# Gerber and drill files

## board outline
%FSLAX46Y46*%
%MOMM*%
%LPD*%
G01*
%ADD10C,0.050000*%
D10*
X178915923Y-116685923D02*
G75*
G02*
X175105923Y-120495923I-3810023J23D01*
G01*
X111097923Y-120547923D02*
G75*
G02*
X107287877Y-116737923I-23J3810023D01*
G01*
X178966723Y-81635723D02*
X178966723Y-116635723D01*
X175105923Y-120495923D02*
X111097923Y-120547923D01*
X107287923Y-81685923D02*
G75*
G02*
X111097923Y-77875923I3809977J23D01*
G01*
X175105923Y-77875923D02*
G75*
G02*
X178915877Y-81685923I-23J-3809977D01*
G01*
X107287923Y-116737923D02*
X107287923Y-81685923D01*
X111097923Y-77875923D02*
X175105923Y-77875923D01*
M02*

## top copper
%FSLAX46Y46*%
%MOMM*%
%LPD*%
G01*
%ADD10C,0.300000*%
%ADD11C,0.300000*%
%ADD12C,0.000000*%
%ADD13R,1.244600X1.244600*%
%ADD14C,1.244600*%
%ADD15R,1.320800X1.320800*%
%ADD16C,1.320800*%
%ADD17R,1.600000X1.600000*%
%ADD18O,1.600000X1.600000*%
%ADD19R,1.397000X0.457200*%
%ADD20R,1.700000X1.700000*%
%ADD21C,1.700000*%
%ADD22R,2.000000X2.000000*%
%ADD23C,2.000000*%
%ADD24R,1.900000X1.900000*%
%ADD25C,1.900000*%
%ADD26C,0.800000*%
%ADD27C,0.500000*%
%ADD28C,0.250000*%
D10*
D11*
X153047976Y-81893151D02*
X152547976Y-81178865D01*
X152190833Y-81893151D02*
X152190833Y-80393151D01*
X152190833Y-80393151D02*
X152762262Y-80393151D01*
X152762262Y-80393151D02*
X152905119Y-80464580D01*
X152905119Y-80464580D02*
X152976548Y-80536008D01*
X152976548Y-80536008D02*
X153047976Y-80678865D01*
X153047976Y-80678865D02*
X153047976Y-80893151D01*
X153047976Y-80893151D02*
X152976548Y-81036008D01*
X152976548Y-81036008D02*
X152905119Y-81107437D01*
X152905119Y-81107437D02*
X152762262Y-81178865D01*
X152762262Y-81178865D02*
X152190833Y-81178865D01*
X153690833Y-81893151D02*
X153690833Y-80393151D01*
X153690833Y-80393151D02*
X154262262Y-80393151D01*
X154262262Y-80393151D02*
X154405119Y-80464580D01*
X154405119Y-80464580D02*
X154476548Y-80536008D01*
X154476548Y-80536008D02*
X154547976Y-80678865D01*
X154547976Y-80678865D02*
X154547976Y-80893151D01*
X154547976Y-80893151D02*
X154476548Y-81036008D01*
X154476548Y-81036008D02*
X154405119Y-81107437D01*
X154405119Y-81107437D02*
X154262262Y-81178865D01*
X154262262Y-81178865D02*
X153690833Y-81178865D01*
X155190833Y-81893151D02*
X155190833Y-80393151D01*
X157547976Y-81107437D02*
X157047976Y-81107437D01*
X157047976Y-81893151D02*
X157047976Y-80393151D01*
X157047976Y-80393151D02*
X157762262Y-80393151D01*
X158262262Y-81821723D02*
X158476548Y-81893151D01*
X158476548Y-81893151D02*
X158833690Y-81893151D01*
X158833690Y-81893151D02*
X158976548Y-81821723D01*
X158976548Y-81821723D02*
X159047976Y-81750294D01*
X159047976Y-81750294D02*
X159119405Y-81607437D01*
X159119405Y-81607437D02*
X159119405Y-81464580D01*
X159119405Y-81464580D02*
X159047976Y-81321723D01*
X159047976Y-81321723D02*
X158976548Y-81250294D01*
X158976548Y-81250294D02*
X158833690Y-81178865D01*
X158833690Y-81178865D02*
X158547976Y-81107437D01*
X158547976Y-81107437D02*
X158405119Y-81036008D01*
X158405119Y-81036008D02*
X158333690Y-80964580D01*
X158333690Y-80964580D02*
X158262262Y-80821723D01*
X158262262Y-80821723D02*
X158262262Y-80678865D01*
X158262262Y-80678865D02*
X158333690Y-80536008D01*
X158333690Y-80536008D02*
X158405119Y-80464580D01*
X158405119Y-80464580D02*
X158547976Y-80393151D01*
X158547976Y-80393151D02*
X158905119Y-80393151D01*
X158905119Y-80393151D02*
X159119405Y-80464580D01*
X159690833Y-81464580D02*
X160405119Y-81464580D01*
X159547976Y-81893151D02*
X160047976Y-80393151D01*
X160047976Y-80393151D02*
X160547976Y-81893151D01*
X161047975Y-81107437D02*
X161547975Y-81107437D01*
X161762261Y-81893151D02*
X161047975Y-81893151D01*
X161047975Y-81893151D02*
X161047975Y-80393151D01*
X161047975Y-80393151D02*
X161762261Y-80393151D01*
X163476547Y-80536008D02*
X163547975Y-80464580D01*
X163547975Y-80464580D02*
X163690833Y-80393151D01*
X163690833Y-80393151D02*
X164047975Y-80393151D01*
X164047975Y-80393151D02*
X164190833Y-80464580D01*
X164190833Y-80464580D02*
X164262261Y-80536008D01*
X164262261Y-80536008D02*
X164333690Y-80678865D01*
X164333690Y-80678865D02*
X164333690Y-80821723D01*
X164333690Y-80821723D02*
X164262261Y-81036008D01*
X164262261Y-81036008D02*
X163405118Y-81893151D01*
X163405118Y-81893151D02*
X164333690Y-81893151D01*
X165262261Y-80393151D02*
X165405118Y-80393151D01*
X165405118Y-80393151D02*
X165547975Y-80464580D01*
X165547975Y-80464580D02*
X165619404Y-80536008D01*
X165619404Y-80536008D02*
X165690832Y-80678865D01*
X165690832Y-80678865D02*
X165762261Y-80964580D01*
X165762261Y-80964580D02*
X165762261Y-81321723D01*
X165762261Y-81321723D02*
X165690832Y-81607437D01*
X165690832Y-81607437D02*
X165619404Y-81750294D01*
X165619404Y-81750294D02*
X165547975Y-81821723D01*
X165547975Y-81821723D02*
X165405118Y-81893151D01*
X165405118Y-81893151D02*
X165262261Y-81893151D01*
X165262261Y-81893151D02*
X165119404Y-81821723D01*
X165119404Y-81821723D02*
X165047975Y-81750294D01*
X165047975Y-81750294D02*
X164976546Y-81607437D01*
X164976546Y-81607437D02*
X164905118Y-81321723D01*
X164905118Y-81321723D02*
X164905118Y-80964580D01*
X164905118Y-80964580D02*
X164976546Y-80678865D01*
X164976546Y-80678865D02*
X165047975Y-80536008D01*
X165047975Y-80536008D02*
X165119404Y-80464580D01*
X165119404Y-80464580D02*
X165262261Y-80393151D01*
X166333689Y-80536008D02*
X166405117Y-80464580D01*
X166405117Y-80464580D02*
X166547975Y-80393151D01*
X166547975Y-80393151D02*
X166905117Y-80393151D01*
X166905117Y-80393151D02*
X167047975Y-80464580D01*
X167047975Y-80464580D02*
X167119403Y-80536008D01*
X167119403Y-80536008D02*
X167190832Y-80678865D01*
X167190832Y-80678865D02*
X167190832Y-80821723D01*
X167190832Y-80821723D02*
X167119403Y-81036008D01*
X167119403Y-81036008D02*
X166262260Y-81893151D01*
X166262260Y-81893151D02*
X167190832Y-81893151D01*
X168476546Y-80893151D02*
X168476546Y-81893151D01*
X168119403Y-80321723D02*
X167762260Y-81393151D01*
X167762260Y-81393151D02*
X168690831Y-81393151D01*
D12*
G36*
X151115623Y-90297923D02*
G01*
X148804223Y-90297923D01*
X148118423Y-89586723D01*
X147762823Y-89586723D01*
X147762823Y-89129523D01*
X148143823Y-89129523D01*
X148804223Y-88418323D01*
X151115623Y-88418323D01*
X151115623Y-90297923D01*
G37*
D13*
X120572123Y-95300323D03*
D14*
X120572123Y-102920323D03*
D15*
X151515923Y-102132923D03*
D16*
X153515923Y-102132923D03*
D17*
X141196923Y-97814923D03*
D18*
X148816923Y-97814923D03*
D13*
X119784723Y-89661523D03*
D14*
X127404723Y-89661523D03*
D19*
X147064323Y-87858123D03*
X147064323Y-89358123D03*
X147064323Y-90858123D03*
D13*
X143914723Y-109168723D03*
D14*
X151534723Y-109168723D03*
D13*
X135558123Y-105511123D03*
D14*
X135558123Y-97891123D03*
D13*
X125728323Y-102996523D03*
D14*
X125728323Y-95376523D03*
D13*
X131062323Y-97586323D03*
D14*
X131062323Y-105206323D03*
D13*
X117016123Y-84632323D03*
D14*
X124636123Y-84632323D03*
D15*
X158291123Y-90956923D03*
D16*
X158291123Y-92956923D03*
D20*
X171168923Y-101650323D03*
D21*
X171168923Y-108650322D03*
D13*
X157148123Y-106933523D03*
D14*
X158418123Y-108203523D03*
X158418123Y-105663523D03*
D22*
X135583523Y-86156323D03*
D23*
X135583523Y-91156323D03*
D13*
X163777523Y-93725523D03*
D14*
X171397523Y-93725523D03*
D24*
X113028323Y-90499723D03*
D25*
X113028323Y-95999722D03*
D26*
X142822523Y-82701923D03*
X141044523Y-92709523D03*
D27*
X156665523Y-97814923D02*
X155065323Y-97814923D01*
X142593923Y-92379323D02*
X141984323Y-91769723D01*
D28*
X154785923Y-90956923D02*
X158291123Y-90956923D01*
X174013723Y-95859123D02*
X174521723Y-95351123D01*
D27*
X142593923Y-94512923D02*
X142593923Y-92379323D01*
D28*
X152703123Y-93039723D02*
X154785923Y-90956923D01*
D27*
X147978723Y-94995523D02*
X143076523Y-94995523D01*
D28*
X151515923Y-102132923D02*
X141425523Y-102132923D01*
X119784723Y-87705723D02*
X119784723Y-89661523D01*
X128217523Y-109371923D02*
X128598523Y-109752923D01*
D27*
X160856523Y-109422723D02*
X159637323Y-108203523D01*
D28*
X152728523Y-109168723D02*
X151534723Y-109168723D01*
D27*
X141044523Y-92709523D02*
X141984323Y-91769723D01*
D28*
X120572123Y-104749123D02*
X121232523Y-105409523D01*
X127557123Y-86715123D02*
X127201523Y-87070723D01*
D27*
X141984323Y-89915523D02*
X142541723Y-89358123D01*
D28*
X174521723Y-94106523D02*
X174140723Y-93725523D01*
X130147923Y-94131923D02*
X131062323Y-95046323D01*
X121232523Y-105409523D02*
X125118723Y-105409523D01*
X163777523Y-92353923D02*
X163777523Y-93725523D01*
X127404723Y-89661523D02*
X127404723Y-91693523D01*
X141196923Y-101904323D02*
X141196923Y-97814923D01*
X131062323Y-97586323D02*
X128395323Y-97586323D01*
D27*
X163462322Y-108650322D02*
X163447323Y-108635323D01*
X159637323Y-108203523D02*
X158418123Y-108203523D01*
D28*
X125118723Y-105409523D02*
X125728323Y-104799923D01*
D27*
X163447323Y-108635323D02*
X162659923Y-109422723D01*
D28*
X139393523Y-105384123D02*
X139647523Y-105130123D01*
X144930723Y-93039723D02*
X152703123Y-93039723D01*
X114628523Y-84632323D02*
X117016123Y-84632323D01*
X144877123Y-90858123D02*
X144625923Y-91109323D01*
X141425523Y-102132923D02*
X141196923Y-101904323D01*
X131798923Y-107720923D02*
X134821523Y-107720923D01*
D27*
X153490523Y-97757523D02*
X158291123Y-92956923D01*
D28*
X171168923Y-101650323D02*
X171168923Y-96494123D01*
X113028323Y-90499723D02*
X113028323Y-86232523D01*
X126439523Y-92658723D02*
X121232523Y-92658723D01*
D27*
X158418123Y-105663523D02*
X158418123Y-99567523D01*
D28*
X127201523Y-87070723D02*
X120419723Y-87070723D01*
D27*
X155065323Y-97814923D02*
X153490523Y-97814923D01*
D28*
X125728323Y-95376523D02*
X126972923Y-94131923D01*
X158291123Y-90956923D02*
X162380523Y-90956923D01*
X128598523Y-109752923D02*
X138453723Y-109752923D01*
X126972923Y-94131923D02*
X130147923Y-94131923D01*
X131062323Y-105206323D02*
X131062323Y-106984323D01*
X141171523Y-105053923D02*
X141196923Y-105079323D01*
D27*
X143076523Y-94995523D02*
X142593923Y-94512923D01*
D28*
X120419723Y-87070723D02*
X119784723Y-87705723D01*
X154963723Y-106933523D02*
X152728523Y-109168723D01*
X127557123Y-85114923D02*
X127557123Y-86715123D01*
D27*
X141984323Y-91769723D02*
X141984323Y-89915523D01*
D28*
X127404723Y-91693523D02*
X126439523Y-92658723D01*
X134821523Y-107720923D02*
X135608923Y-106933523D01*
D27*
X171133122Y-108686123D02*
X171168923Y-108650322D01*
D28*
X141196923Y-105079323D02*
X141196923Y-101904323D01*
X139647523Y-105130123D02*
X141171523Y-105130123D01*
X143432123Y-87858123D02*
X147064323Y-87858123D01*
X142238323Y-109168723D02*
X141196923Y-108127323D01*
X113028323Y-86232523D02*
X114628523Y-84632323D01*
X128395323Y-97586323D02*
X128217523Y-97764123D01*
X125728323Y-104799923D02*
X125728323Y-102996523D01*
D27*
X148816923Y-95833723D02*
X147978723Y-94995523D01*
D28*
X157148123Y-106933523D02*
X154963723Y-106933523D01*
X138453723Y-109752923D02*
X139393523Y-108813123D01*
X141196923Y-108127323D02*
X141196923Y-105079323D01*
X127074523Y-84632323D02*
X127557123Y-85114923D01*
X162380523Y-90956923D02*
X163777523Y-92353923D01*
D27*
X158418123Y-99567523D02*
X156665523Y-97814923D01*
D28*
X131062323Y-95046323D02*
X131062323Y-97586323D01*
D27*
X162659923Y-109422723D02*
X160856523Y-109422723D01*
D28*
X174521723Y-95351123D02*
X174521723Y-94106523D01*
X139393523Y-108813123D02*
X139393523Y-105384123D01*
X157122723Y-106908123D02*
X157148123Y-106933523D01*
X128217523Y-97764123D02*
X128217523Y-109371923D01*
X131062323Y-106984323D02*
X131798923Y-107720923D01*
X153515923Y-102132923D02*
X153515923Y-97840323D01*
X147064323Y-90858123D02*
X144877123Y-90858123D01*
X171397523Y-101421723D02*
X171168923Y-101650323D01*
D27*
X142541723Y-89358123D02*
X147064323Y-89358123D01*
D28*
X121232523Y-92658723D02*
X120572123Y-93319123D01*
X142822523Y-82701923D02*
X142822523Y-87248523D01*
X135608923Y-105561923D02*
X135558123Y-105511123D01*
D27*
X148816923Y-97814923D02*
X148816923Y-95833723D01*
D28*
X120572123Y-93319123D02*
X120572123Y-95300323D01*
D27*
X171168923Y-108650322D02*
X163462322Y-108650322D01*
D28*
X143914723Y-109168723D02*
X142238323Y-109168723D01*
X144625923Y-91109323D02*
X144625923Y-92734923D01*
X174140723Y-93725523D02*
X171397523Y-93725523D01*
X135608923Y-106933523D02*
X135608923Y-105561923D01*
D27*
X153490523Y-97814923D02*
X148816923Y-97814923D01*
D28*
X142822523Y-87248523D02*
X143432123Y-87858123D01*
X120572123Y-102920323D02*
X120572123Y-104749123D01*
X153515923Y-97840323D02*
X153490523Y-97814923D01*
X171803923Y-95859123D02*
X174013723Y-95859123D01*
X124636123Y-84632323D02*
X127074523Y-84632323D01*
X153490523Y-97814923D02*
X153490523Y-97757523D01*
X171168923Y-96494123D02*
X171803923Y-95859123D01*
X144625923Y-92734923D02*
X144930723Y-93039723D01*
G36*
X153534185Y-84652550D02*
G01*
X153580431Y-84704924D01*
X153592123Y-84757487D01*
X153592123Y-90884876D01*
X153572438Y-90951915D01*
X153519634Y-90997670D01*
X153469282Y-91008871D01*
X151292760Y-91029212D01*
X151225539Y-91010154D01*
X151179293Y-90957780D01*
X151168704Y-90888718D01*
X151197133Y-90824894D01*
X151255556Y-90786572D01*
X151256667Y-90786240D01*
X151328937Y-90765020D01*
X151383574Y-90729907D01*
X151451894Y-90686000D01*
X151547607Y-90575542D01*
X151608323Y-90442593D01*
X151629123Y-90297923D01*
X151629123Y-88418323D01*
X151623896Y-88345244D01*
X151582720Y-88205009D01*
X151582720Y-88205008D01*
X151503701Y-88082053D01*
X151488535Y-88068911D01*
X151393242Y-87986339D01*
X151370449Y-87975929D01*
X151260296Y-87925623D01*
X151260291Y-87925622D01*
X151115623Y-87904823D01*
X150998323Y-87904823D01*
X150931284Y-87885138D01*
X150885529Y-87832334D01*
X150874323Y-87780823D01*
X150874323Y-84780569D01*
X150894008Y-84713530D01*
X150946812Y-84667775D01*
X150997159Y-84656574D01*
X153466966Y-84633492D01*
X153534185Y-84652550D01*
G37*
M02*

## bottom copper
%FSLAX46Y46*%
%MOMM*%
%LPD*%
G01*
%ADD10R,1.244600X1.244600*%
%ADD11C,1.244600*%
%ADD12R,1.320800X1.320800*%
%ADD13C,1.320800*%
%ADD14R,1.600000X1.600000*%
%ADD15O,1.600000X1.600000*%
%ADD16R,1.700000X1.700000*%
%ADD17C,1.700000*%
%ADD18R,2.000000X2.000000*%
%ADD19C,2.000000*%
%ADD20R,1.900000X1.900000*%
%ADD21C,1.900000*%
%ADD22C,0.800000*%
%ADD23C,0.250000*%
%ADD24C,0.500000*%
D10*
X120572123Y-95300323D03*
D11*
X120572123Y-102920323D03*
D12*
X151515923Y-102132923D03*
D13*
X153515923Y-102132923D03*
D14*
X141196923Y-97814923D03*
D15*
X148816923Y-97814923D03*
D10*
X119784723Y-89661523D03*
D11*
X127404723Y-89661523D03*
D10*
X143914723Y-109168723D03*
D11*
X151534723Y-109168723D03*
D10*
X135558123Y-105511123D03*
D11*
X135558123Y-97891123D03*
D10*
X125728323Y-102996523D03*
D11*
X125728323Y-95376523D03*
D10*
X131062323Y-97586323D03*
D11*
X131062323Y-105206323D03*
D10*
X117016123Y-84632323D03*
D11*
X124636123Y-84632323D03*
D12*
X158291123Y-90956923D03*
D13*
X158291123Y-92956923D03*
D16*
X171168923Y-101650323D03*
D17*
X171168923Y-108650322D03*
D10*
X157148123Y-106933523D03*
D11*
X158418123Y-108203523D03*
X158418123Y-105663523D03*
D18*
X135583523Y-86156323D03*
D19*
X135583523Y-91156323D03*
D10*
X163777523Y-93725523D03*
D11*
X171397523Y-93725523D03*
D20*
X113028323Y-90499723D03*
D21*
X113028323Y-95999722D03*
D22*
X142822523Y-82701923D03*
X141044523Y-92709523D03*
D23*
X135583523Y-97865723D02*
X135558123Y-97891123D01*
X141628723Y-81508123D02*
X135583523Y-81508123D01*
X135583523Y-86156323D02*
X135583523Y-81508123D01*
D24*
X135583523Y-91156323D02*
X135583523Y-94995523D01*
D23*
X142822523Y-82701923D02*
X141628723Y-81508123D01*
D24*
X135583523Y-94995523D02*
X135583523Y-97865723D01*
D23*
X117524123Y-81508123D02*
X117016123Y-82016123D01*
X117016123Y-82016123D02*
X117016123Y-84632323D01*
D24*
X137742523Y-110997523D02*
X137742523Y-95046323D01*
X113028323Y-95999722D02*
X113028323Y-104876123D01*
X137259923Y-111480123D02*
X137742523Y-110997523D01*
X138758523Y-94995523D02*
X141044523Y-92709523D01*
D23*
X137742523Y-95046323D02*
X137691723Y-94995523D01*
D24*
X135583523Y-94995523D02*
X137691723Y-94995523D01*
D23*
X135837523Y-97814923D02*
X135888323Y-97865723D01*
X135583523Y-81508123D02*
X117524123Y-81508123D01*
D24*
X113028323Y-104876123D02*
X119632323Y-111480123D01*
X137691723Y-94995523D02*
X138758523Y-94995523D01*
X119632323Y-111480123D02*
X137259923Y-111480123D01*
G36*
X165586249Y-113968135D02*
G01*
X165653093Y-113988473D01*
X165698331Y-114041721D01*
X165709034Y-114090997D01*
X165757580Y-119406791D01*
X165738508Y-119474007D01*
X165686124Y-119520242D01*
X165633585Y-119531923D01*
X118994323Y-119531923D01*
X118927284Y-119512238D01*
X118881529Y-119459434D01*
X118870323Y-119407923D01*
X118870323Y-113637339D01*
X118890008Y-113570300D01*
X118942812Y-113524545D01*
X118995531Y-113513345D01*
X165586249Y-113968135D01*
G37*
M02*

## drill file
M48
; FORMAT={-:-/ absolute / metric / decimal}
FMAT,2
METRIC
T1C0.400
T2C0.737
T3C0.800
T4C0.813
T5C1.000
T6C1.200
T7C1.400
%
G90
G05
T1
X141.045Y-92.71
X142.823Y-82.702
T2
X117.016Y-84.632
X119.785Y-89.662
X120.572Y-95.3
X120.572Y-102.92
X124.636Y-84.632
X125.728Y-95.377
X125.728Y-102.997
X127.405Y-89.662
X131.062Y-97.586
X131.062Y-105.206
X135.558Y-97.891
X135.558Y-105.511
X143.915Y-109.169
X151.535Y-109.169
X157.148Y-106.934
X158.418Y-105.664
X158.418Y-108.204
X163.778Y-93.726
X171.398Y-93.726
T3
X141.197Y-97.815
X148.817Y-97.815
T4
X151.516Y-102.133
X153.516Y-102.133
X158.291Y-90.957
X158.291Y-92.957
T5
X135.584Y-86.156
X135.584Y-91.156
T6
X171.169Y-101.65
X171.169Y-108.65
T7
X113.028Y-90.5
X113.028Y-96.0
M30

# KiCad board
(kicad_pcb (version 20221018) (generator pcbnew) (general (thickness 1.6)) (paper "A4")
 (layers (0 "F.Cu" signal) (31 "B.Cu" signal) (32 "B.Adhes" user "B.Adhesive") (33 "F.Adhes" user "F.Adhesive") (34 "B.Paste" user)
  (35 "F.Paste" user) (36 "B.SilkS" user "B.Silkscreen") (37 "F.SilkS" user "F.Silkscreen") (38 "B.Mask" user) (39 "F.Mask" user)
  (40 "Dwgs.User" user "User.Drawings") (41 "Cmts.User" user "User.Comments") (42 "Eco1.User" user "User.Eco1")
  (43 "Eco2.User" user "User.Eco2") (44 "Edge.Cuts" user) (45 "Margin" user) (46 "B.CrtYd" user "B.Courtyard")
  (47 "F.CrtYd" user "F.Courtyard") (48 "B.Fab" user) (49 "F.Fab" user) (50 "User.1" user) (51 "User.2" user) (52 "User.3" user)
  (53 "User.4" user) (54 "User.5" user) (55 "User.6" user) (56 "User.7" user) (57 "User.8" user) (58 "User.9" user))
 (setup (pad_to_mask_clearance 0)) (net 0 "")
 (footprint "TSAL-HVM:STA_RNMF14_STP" (layer "F.Cu") (at 120.572123 95.300323 -90)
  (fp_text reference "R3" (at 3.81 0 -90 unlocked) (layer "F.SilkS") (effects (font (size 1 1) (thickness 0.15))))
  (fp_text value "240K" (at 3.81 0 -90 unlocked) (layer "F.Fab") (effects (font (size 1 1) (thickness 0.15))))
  (pad "1" thru_hole rect (at 0 0 270) (size 1.2446 1.2446) (drill 0.7366) (layers "*.Cu" "*.Mask"))
  (pad "2" thru_hole circle (at 7.62 0 270) (size 1.2446 1.2446) (drill 0.7366) (layers "*.Cu" "*.Mask")))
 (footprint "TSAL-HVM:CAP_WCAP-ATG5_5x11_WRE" (layer "F.Cu") (at 151.515923 102.132923)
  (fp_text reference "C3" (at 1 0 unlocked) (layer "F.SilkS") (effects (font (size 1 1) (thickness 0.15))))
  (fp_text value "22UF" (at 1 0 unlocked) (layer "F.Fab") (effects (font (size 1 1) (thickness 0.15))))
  (pad "1" thru_hole rect (at 0 0) (size 1.3208 1.3208) (drill 0.8128) (layers "*.Cu" "*.Mask"))
  (pad "2" thru_hole circle (at 2 0) (size 1.3208 1.3208) (drill 0.8128) (layers "*.Cu" "*.Mask")))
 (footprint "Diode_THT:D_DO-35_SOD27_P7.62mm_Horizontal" (layer "F.Cu") (at 141.196923 97.814923)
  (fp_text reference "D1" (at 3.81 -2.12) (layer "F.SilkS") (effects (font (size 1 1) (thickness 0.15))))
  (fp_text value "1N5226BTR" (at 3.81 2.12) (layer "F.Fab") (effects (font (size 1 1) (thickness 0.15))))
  (pad "1" thru_hole rect (at 0 0) (size 1.6 1.6) (drill 0.8) (layers "*.Cu" "*.Mask"))
  (pad "2" thru_hole oval (at 7.62 0) (size 1.6 1.6) (drill 0.8) (layers "*.Cu" "*.Mask")))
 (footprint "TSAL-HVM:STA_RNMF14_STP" (layer "F.Cu") (at 119.784723 89.661523)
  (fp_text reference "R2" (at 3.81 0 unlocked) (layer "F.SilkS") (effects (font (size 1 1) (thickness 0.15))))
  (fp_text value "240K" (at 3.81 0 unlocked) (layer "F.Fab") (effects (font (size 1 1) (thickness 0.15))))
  (pad "1" thru_hole rect (at 0 0) (size 1.2446 1.2446) (drill 0.7366) (layers "*.Cu" "*.Mask"))
  (pad "2" thru_hole circle (at 7.62 0) (size 1.2446 1.2446) (drill 0.7366) (layers "*.Cu" "*.Mask")))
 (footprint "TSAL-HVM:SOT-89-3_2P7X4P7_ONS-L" (layer "F.Cu") (at 149.109023 89.358123 -90)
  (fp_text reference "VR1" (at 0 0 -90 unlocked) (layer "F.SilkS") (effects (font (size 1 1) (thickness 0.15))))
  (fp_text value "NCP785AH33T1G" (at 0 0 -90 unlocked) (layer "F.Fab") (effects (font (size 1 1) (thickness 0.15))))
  (fp_poly
   (pts (xy -0.2286 1.3462) (xy -0.2286 0.9652) (xy -0.9398 0.3048) (xy -0.9398 -2.0066) (xy 0.9398 -2.0066) (xy 0.9398 0.3048)
    (xy 0.2286 0.9906) (xy 0.2286 1.3462))
   (stroke (width 0) (type solid)) (fill solid) (layer "F.Cu"))
  (pad "1" smd rect (at -1.5 2.0447 270) (size 0.4572 1.397) (layers "F.Cu" "F.Paste" "F.Mask"))
  (pad "2" smd rect (at 0 2.0447 270) (size 0.4572 1.397) (layers "F.Cu" "F.Paste" "F.Mask"))
  (pad "3" smd rect (at 1.5 2.0447 270) (size 0.4572 1.397) (layers "F.Cu" "F.Paste" "F.Mask")))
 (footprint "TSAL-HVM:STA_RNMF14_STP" (layer "F.Cu") (at 143.914723 109.168723)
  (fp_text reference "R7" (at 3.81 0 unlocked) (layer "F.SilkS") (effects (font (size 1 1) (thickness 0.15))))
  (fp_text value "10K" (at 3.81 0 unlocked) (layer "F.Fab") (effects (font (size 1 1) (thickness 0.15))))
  (pad "1" thru_hole rect (at 0 0) (size 1.2446 1.2446) (drill 0.7366) (layers "*.Cu" "*.Mask"))
  (pad "2" thru_hole circle (at 7.62 0) (size 1.2446 1.2446) (drill 0.7366) (layers "*.Cu" "*.Mask")))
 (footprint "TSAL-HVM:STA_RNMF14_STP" (layer "F.Cu") (at 135.558123 105.511123 90)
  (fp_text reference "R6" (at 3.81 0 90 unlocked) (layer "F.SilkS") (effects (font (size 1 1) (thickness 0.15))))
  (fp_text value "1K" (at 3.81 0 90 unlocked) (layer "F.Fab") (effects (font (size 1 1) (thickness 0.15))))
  (pad "1" thru_hole rect (at 0 0 90) (size 1.2446 1.2446) (drill 0.7366) (layers "*.Cu" "*.Mask"))
  (pad "2" thru_hole circle (at 7.62 0 90) (size 1.2446 1.2446) (drill 0.7366) (layers "*.Cu" "*.Mask")))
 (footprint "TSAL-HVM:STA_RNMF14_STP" (layer "F.Cu") (at 125.728323 102.996523 90)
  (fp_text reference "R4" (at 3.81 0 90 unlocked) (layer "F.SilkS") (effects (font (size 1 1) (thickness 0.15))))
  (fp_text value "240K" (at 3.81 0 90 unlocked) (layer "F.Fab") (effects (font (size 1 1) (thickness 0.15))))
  (pad "1" thru_hole rect (at 0 0 90) (size 1.2446 1.2446) (drill 0.7366) (layers "*.Cu" "*.Mask"))
  (pad "2" thru_hole circle (at 7.62 0 90) (size 1.2446 1.2446) (drill 0.7366) (layers "*.Cu" "*.Mask")))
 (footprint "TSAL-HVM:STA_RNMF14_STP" (layer "F.Cu") (at 131.062323 97.586323 -90)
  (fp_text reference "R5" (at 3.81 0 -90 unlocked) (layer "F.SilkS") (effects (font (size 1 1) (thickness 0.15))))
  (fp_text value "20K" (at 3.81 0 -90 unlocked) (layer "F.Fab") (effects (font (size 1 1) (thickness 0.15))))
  (pad "1" thru_hole rect (at 0 0 270) (size 1.2446 1.2446) (drill 0.7366) (layers "*.Cu" "*.Mask"))
  (pad "2" thru_hole circle (at 7.62 0 270) (size 1.2446 1.2446) (drill 0.7366) (layers "*.Cu" "*.Mask")))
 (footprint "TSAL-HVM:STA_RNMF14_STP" (layer "F.Cu") (at 117.016123 84.632323)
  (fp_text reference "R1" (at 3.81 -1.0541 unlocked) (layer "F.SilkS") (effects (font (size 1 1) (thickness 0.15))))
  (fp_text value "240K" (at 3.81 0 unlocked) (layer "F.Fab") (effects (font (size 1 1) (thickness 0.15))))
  (pad "1" thru_hole rect (at 0 0) (size 1.2446 1.2446) (drill 0.7366) (layers "*.Cu" "*.Mask"))
  (pad "2" thru_hole circle (at 7.62 0) (size 1.2446 1.2446) (drill 0.7366) (layers "*.Cu" "*.Mask")))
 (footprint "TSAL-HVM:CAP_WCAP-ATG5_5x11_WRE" (layer "F.Cu") (at 158.291123 90.956923 -90)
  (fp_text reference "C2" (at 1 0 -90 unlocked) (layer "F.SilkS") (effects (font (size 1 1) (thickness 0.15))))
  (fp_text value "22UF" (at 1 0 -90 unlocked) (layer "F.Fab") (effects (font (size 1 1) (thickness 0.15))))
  (pad "1" thru_hole rect (at 0 0 270) (size 1.3208 1.3208) (drill 0.8128) (layers "*.Cu" "*.Mask"))
  (pad "2" thru_hole circle (at 2 0 270) (size 1.3208 1.3208) (drill 0.8128) (layers "*.Cu" "*.Mask")))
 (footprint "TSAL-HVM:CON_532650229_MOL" (layer "F.Cu") (at 171.168923 101.650323 90)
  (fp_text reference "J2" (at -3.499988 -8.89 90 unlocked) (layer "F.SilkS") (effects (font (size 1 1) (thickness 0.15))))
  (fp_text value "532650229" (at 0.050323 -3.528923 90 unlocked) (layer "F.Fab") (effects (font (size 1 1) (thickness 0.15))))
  (pad "1" thru_hole rect (at 0 0 90) (size 1.7 1.7) (drill 1.2) (layers "*.Cu" "*.Mask"))
  (pad "2" thru_hole circle (at -6.999999 0 90) (size 1.7 1.7) (drill 1.2) (layers "*.Cu" "*.Mask")))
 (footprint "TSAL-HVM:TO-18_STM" (layer "F.Cu") (at 157.148123 106.933523)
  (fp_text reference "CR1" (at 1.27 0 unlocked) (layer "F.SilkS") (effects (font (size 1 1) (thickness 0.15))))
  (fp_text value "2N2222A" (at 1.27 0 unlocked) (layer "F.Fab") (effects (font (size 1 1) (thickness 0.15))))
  (pad "1" thru_hole rect (at 0 0) (size 1.2446 1.2446) (drill 0.7366) (layers "*.Cu" "*.Mask"))
  (pad "2" thru_hole circle (at 1.27 1.27) (size 1.2446 1.2446) (drill 0.7366) (layers "*.Cu" "*.Mask"))
  (pad "3" thru_hole circle (at 1.27 -1.27) (size 1.2446 1.2446) (drill 0.7366) (layers "*.Cu" "*.Mask")))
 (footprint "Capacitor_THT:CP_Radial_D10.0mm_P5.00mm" (layer "F.Cu") (at 135.583523 86.156323 -90)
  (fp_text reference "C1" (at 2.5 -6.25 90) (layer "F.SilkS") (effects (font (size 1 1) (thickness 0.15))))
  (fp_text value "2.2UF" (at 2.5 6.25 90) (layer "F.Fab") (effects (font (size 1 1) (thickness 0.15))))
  (pad "1" thru_hole rect (at 0 0 270) (size 2 2) (drill 1) (layers "*.Cu" "*.Mask"))
  (pad "2" thru_hole circle (at 5 0 270) (size 2 2) (drill 1) (layers "*.Cu" "*.Mask")))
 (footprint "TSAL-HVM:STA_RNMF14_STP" (layer "F.Cu") (at 163.777523 93.725523)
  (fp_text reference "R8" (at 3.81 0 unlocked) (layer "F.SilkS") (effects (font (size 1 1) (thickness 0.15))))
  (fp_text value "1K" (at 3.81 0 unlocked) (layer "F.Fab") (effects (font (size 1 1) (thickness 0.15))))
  (pad "1" thru_hole rect (at 0 0) (size 1.2446 1.2446) (drill 0.7366) (layers "*.Cu" "*.Mask"))
  (pad "2" thru_hole circle (at 7.62 0) (size 1.2446 1.2446) (drill 0.7366) (layers "*.Cu" "*.Mask")))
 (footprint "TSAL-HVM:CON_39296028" (layer "F.Cu") (at 113.028323 90.499723)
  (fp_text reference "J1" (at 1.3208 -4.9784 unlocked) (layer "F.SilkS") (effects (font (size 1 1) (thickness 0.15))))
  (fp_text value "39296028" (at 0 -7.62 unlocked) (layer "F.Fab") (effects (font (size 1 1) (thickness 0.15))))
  (pad "1" thru_hole rect (at 0 0) (size 1.9 1.9) (drill 1.4) (layers "*.Cu" "*.Mask"))
  (pad "2" thru_hole circle (at 0 5.499999) (size 1.9 1.9) (drill 1.4) (layers "*.Cu" "*.Mask")))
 (gr_arc (start 178.915923 116.685923) (mid 177.8 119.38) (end 175.105923 120.495923) (stroke (width 0.05) (type solid)) (layer "Edge.Cuts"))
 (gr_arc (start 111.097923 120.547923) (mid 108.403846 119.432) (end 107.287923 116.737923) (stroke (width 0.05) (type solid))
  (layer "Edge.Cuts"))
 (gr_line (start 178.966723 81.635723) (end 178.966723 116.635723) (stroke (width 0.05) (type solid)) (layer "Edge.Cuts"))
 (gr_line (start 175.105923 120.495923) (end 111.097923 120.547923) (stroke (width 0.05) (type solid)) (layer "Edge.Cuts"))
 (gr_arc (start 107.287923 81.685923) (mid 108.403846 78.991846) (end 111.097923 77.875923) (stroke (width 0.05) (type solid))
  (layer "Edge.Cuts"))
 (gr_arc (start 175.105923 77.875923) (mid 177.8 78.991846) (end 178.915923 81.685923) (stroke (width 0.05) (type solid))
  (layer "Edge.Cuts"))
 (gr_line (start 107.287923 116.737923) (end 107.287923 81.685923) (stroke (width 0.05) (type solid)) (layer "Edge.Cuts"))
 (gr_line (start 111.097923 77.875923) (end 175.105923 77.875923) (stroke (width 0.05) (type solid)) (layer "Edge.Cuts"))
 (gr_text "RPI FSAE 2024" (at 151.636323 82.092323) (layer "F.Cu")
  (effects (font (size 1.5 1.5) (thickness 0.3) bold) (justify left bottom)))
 (segment (start 156.665523 97.814923) (end 155.065323 97.814923) (width 0.5) (layer "F.Cu") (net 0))
 (segment (start 142.593923 92.379323) (end 141.984323 91.769723) (width 0.5) (layer "F.Cu") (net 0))
 (segment (start 154.785923 90.956923) (end 158.291123 90.956923) (width 0.25) (layer "F.Cu") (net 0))
 (segment (start 174.013723 95.859123) (end 174.521723 95.351123) (width 0.25) (layer "F.Cu") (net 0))
 (segment (start 142.593923 94.512923) (end 142.593923 92.379323) (width 0.5) (layer "F.Cu") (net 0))
 (segment (start 152.703123 93.039723) (end 154.785923 90.956923) (width 0.25) (layer "F.Cu") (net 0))
 (segment (start 147.978723 94.995523) (end 143.076523 94.995523) (width 0.5) (layer "F.Cu") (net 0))
 (segment (start 151.515923 102.132923) (end 141.425523 102.132923) (width 0.25) (layer "F.Cu") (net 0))
 (segment (start 119.784723 87.705723) (end 119.784723 89.661523) (width 0.25) (layer "F.Cu") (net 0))
 (segment (start 128.217523 109.371923) (end 128.598523 109.752923) (width 0.25) (layer "F.Cu") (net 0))
 (segment (start 160.856523 109.422723) (end 159.637323 108.203523) (width 0.5) (layer "F.Cu") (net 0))
 (segment (start 152.728523 109.168723) (end 151.534723 109.168723) (width 0.25) (layer "F.Cu") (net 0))
 (segment (start 141.044523 92.709523) (end 141.984323 91.769723) (width 0.5) (layer "F.Cu") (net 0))
 (segment (start 120.572123 104.749123) (end 121.232523 105.409523) (width 0.25) (layer "F.Cu") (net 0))
 (segment (start 127.557123 86.715123) (end 127.201523 87.070723) (width 0.25) (layer "F.Cu") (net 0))
 (segment (start 141.984323 89.915523) (end 142.541723 89.358123) (width 0.5) (layer "F.Cu") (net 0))
 (segment (start 174.521723 94.106523) (end 174.140723 93.725523) (width 0.25) (layer "F.Cu") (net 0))
 (segment (start 130.147923 94.131923) (end 131.062323 95.046323) (width 0.25) (layer "F.Cu") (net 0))
 (segment (start 121.232523 105.409523) (end 125.118723 105.409523) (width 0.25) (layer "F.Cu") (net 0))
 (segment (start 163.777523 92.353923) (end 163.777523 93.725523) (width 0.25) (layer "F.Cu") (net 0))
 (segment (start 127.404723 89.661523) (end 127.404723 91.693523) (width 0.25) (layer "F.Cu") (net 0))
 (segment (start 141.196923 101.904323) (end 141.196923 97.814923) (width 0.25) (layer "F.Cu") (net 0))
 (segment (start 131.062323 97.586323) (end 128.395323 97.586323) (width 0.25) (layer "F.Cu") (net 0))
 (segment (start 163.462322 108.650322) (end 163.447323 108.635323) (width 0.5) (layer "F.Cu") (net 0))
 (segment (start 159.637323 108.203523) (end 158.418123 108.203523) (width 0.5) (layer "F.Cu") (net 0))
 (segment (start 125.118723 105.409523) (end 125.728323 104.799923) (width 0.25) (layer "F.Cu") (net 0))
 (segment (start 163.447323 108.635323) (end 162.659923 109.422723) (width 0.5) (layer "F.Cu") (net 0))
 (segment (start 139.393523 105.384123) (end 139.647523 105.130123) (width 0.25) (layer "F.Cu") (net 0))
 (segment (start 144.930723 93.039723) (end 152.703123 93.039723) (width 0.25) (layer "F.Cu") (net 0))
 (segment (start 114.628523 84.632323) (end 117.016123 84.632323) (width 0.25) (layer "F.Cu") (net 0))
 (segment (start 144.877123 90.858123) (end 144.625923 91.109323) (width 0.25) (layer "F.Cu") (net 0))
 (segment (start 141.425523 102.132923) (end 141.196923 101.904323) (width 0.25) (layer "F.Cu") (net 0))
 (segment (start 131.798923 107.720923) (end 134.821523 107.720923) (width 0.25) (layer "F.Cu") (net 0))
 (segment (start 153.490523 97.757523) (end 158.291123 92.956923) (width 0.5) (layer "F.Cu") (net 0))
 (segment (start 171.168923 101.650323) (end 171.168923 96.494123) (width 0.25) (layer "F.Cu") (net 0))
 (segment (start 113.028323 90.499723) (end 113.028323 86.232523) (width 0.25) (layer "F.Cu") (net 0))
 (segment (start 126.439523 92.658723) (end 121.232523 92.658723) (width 0.25) (layer "F.Cu") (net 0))
 (segment (start 158.418123 105.663523) (end 158.418123 99.567523) (width 0.5) (layer "F.Cu") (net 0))
 (segment (start 127.201523 87.070723) (end 120.419723 87.070723) (width 0.25) (layer "F.Cu") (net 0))
 (segment (start 155.065323 97.814923) (end 153.490523 97.814923) (width 0.5) (layer "F.Cu") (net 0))
 (segment (start 125.728323 95.376523) (end 126.972923 94.131923) (width 0.25) (layer "F.Cu") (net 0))
 (segment (start 158.291123 90.956923) (end 162.380523 90.956923) (width 0.25) (layer "F.Cu") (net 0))
 (segment (start 128.598523 109.752923) (end 138.453723 109.752923) (width 0.25) (layer "F.Cu") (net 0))
 (segment (start 126.972923 94.131923) (end 130.147923 94.131923) (width 0.25) (layer "F.Cu") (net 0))
 (segment (start 131.062323 105.206323) (end 131.062323 106.984323) (width 0.25) (layer "F.Cu") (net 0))
 (segment (start 141.171523 105.053923) (end 141.196923 105.079323) (width 0.25) (layer "F.Cu") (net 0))
 (segment (start 143.076523 94.995523) (end 142.593923 94.512923) (width 0.5) (layer "F.Cu") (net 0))
 (segment (start 120.419723 87.070723) (end 119.784723 87.705723) (width 0.25) (layer "F.Cu") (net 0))
 (segment (start 154.963723 106.933523) (end 152.728523 109.168723) (width 0.25) (layer "F.Cu") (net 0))
 (segment (start 127.557123 85.114923) (end 127.557123 86.715123) (width 0.25) (layer "F.Cu") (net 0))
 (segment (start 141.984323 91.769723) (end 141.984323 89.915523) (width 0.5) (layer "F.Cu") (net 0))
 (segment (start 127.404723 91.693523) (end 126.439523 92.658723) (width 0.25) (layer "F.Cu") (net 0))
 (segment (start 134.821523 107.720923) (end 135.608923 106.933523) (width 0.25) (layer "F.Cu") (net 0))
 (segment (start 171.133122 108.686123) (end 171.168923 108.650322) (width 0.5) (layer "F.Cu") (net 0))
 (segment (start 141.196923 105.079323) (end 141.196923 101.904323) (width 0.25) (layer "F.Cu") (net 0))
 (segment (start 139.647523 105.130123) (end 141.171523 105.130123) (width 0.25) (layer "F.Cu") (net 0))
 (segment (start 143.432123 87.858123) (end 147.064323 87.858123) (width 0.25) (layer "F.Cu") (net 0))
 (segment (start 142.238323 109.168723) (end 141.196923 108.127323) (width 0.25) (layer "F.Cu") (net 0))
 (segment (start 113.028323 86.232523) (end 114.628523 84.632323) (width 0.25) (layer "F.Cu") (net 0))
 (segment (start 128.395323 97.586323) (end 128.217523 97.764123) (width 0.25) (layer "F.Cu") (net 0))
 (segment (start 125.728323 104.799923) (end 125.728323 102.996523) (width 0.25) (layer "F.Cu") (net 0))
 (segment (start 148.816923 95.833723) (end 147.978723 94.995523) (width 0.5) (layer "F.Cu") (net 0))
 (segment (start 157.148123 106.933523) (end 154.963723 106.933523) (width 0.25) (layer "F.Cu") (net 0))
 (segment (start 138.453723 109.752923) (end 139.393523 108.813123) (width 0.25) (layer "F.Cu") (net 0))
 (segment (start 141.196923 108.127323) (end 141.196923 105.079323) (width 0.25) (layer "F.Cu") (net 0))
 (segment (start 127.074523 84.632323) (end 127.557123 85.114923) (width 0.25) (layer "F.Cu") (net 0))
 (segment (start 162.380523 90.956923) (end 163.777523 92.353923) (width 0.25) (layer "F.Cu") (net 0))
 (segment (start 158.418123 99.567523) (end 156.665523 97.814923) (width 0.5) (layer "F.Cu") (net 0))
 (segment (start 131.062323 95.046323) (end 131.062323 97.586323) (width 0.25) (layer "F.Cu") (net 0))
 (segment (start 162.659923 109.422723) (end 160.856523 109.422723) (width 0.5) (layer "F.Cu") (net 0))
 (segment (start 174.521723 95.351123) (end 174.521723 94.106523) (width 0.25) (layer "F.Cu") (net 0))
 (segment (start 139.393523 108.813123) (end 139.393523 105.384123) (width 0.25) (layer "F.Cu") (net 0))
 (segment (start 157.122723 106.908123) (end 157.148123 106.933523) (width 0.25) (layer "F.Cu") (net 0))
 (segment (start 128.217523 97.764123) (end 128.217523 109.371923) (width 0.25) (layer "F.Cu") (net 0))
 (segment (start 131.062323 106.984323) (end 131.798923 107.720923) (width 0.25) (layer "F.Cu") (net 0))
 (segment (start 153.515923 102.132923) (end 153.515923 97.840323) (width 0.25) (layer "F.Cu") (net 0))
 (segment (start 147.064323 90.858123) (end 144.877123 90.858123) (width 0.25) (layer "F.Cu") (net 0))
 (segment (start 171.397523 101.421723) (end 171.168923 101.650323) (width 0.25) (layer "F.Cu") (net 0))
 (segment (start 142.541723 89.358123) (end 147.064323 89.358123) (width 0.5) (layer "F.Cu") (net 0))
 (segment (start 121.232523 92.658723) (end 120.572123 93.319123) (width 0.25) (layer "F.Cu") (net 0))
 (segment (start 142.822523 82.701923) (end 142.822523 87.248523) (width 0.25) (layer "F.Cu") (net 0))
 (segment (start 135.608923 105.561923) (end 135.558123 105.511123) (width 0.25) (layer "F.Cu") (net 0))
 (segment (start 148.816923 97.814923) (end 148.816923 95.833723) (width 0.5) (layer "F.Cu") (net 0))
 (segment (start 120.572123 93.319123) (end 120.572123 95.300323) (width 0.25) (layer "F.Cu") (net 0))
 (segment (start 171.168923 108.650322) (end 163.462322 108.650322) (width 0.5) (layer "F.Cu") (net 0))
 (segment (start 143.914723 109.168723) (end 142.238323 109.168723) (width 0.25) (layer "F.Cu") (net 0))
 (segment (start 144.625923 91.109323) (end 144.625923 92.734923) (width 0.25) (layer "F.Cu") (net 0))
 (segment (start 174.140723 93.725523) (end 171.397523 93.725523) (width 0.25) (layer "F.Cu") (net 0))
 (segment (start 135.608923 106.933523) (end 135.608923 105.561923) (width 0.25) (layer "F.Cu") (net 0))
 (segment (start 153.490523 97.814923) (end 148.816923 97.814923) (width 0.5) (layer "F.Cu") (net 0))
 (segment (start 142.822523 87.248523) (end 143.432123 87.858123) (width 0.25) (layer "F.Cu") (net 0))
 (segment (start 120.572123 102.920323) (end 120.572123 104.749123) (width 0.25) (layer "F.Cu") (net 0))
 (segment (start 153.515923 97.840323) (end 153.490523 97.814923) (width 0.25) (layer "F.Cu") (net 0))
 (segment (start 171.803923 95.859123) (end 174.013723 95.859123) (width 0.25) (layer "F.Cu") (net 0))
 (segment (start 124.636123 84.632323) (end 127.074523 84.632323) (width 0.25) (layer "F.Cu") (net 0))
 (segment (start 153.490523 97.814923) (end 153.490523 97.757523) (width 0.25) (layer "F.Cu") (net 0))
 (segment (start 171.168923 96.494123) (end 171.803923 95.859123) (width 0.25) (layer "F.Cu") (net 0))
 (segment (start 144.625923 92.734923) (end 144.930723 93.039723) (width 0.25) (layer "F.Cu") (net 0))
 (via (at 142.822523 82.701923) (size 0.8) (drill 0.4) (layers "F.Cu" "B.Cu") (free) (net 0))
 (via (at 141.044523 92.709523) (size 0.8) (drill 0.4) (layers "F.Cu" "B.Cu") (free) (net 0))
 (segment (start 135.583523 97.865723) (end 135.558123 97.891123) (width 0.25) (layer "B.Cu") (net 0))
 (segment (start 141.628723 81.508123) (end 135.583523 81.508123) (width 0.25) (layer "B.Cu") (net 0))
 (segment (start 135.583523 86.156323) (end 135.583523 81.508123) (width 0.25) (layer "B.Cu") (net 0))
 (segment (start 135.583523 91.156323) (end 135.583523 94.995523) (width 0.5) (layer "B.Cu") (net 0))
 (segment (start 142.822523 82.701923) (end 141.628723 81.508123) (width 0.25) (layer "B.Cu") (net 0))
 (segment (start 135.583523 94.995523) (end 135.583523 97.865723) (width 0.5) (layer "B.Cu") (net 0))
 (segment (start 117.524123 81.508123) (end 117.016123 82.016123) (width 0.25) (layer "B.Cu") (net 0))
 (segment (start 117.016123 82.016123) (end 117.016123 84.632323) (width 0.25) (layer "B.Cu") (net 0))
 (segment (start 137.742523 110.997523) (end 137.742523 95.046323) (width 0.5) (layer "B.Cu") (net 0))
 (segment (start 113.028323 95.999722) (end 113.028323 104.876123) (width 0.5) (layer "B.Cu") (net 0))
 (segment (start 137.259923 111.480123) (end 137.742523 110.997523) (width 0.5) (layer "B.Cu") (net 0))
 (segment (start 138.758523 94.995523) (end 141.044523 92.709523) (width 0.5) (layer "B.Cu") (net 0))
 (segment (start 137.742523 95.046323) (end 137.691723 94.995523) (width 0.25) (layer "B.Cu") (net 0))
 (segment (start 135.583523 94.995523) (end 137.691723 94.995523) (width 0.5) (layer "B.Cu") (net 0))
 (segment (start 135.837523 97.814923) (end 135.888323 97.865723) (width 0.25) (layer "B.Cu") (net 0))
 (segment (start 135.583523 81.508123) (end 117.524123 81.508123) (width 0.25) (layer "B.Cu") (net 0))
 (segment (start 113.028323 104.876123) (end 119.632323 111.480123) (width 0.5) (layer "B.Cu") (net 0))
 (segment (start 137.691723 94.995523) (end 138.758523 94.995523) (width 0.5) (layer "B.Cu") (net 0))
 (segment (start 119.632323 111.480123) (end 137.259923 111.480123) (width 0.5) (layer "B.Cu") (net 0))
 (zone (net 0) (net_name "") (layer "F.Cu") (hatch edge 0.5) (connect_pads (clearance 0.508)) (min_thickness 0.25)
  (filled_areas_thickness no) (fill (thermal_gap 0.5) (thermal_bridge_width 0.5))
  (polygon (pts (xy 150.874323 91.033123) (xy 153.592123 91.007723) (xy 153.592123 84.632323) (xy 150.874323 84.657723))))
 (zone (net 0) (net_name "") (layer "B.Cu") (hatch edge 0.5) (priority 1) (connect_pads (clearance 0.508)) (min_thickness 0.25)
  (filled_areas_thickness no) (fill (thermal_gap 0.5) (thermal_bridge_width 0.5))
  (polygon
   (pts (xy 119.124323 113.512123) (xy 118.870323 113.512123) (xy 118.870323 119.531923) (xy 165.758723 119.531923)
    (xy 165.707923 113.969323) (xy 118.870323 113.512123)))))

